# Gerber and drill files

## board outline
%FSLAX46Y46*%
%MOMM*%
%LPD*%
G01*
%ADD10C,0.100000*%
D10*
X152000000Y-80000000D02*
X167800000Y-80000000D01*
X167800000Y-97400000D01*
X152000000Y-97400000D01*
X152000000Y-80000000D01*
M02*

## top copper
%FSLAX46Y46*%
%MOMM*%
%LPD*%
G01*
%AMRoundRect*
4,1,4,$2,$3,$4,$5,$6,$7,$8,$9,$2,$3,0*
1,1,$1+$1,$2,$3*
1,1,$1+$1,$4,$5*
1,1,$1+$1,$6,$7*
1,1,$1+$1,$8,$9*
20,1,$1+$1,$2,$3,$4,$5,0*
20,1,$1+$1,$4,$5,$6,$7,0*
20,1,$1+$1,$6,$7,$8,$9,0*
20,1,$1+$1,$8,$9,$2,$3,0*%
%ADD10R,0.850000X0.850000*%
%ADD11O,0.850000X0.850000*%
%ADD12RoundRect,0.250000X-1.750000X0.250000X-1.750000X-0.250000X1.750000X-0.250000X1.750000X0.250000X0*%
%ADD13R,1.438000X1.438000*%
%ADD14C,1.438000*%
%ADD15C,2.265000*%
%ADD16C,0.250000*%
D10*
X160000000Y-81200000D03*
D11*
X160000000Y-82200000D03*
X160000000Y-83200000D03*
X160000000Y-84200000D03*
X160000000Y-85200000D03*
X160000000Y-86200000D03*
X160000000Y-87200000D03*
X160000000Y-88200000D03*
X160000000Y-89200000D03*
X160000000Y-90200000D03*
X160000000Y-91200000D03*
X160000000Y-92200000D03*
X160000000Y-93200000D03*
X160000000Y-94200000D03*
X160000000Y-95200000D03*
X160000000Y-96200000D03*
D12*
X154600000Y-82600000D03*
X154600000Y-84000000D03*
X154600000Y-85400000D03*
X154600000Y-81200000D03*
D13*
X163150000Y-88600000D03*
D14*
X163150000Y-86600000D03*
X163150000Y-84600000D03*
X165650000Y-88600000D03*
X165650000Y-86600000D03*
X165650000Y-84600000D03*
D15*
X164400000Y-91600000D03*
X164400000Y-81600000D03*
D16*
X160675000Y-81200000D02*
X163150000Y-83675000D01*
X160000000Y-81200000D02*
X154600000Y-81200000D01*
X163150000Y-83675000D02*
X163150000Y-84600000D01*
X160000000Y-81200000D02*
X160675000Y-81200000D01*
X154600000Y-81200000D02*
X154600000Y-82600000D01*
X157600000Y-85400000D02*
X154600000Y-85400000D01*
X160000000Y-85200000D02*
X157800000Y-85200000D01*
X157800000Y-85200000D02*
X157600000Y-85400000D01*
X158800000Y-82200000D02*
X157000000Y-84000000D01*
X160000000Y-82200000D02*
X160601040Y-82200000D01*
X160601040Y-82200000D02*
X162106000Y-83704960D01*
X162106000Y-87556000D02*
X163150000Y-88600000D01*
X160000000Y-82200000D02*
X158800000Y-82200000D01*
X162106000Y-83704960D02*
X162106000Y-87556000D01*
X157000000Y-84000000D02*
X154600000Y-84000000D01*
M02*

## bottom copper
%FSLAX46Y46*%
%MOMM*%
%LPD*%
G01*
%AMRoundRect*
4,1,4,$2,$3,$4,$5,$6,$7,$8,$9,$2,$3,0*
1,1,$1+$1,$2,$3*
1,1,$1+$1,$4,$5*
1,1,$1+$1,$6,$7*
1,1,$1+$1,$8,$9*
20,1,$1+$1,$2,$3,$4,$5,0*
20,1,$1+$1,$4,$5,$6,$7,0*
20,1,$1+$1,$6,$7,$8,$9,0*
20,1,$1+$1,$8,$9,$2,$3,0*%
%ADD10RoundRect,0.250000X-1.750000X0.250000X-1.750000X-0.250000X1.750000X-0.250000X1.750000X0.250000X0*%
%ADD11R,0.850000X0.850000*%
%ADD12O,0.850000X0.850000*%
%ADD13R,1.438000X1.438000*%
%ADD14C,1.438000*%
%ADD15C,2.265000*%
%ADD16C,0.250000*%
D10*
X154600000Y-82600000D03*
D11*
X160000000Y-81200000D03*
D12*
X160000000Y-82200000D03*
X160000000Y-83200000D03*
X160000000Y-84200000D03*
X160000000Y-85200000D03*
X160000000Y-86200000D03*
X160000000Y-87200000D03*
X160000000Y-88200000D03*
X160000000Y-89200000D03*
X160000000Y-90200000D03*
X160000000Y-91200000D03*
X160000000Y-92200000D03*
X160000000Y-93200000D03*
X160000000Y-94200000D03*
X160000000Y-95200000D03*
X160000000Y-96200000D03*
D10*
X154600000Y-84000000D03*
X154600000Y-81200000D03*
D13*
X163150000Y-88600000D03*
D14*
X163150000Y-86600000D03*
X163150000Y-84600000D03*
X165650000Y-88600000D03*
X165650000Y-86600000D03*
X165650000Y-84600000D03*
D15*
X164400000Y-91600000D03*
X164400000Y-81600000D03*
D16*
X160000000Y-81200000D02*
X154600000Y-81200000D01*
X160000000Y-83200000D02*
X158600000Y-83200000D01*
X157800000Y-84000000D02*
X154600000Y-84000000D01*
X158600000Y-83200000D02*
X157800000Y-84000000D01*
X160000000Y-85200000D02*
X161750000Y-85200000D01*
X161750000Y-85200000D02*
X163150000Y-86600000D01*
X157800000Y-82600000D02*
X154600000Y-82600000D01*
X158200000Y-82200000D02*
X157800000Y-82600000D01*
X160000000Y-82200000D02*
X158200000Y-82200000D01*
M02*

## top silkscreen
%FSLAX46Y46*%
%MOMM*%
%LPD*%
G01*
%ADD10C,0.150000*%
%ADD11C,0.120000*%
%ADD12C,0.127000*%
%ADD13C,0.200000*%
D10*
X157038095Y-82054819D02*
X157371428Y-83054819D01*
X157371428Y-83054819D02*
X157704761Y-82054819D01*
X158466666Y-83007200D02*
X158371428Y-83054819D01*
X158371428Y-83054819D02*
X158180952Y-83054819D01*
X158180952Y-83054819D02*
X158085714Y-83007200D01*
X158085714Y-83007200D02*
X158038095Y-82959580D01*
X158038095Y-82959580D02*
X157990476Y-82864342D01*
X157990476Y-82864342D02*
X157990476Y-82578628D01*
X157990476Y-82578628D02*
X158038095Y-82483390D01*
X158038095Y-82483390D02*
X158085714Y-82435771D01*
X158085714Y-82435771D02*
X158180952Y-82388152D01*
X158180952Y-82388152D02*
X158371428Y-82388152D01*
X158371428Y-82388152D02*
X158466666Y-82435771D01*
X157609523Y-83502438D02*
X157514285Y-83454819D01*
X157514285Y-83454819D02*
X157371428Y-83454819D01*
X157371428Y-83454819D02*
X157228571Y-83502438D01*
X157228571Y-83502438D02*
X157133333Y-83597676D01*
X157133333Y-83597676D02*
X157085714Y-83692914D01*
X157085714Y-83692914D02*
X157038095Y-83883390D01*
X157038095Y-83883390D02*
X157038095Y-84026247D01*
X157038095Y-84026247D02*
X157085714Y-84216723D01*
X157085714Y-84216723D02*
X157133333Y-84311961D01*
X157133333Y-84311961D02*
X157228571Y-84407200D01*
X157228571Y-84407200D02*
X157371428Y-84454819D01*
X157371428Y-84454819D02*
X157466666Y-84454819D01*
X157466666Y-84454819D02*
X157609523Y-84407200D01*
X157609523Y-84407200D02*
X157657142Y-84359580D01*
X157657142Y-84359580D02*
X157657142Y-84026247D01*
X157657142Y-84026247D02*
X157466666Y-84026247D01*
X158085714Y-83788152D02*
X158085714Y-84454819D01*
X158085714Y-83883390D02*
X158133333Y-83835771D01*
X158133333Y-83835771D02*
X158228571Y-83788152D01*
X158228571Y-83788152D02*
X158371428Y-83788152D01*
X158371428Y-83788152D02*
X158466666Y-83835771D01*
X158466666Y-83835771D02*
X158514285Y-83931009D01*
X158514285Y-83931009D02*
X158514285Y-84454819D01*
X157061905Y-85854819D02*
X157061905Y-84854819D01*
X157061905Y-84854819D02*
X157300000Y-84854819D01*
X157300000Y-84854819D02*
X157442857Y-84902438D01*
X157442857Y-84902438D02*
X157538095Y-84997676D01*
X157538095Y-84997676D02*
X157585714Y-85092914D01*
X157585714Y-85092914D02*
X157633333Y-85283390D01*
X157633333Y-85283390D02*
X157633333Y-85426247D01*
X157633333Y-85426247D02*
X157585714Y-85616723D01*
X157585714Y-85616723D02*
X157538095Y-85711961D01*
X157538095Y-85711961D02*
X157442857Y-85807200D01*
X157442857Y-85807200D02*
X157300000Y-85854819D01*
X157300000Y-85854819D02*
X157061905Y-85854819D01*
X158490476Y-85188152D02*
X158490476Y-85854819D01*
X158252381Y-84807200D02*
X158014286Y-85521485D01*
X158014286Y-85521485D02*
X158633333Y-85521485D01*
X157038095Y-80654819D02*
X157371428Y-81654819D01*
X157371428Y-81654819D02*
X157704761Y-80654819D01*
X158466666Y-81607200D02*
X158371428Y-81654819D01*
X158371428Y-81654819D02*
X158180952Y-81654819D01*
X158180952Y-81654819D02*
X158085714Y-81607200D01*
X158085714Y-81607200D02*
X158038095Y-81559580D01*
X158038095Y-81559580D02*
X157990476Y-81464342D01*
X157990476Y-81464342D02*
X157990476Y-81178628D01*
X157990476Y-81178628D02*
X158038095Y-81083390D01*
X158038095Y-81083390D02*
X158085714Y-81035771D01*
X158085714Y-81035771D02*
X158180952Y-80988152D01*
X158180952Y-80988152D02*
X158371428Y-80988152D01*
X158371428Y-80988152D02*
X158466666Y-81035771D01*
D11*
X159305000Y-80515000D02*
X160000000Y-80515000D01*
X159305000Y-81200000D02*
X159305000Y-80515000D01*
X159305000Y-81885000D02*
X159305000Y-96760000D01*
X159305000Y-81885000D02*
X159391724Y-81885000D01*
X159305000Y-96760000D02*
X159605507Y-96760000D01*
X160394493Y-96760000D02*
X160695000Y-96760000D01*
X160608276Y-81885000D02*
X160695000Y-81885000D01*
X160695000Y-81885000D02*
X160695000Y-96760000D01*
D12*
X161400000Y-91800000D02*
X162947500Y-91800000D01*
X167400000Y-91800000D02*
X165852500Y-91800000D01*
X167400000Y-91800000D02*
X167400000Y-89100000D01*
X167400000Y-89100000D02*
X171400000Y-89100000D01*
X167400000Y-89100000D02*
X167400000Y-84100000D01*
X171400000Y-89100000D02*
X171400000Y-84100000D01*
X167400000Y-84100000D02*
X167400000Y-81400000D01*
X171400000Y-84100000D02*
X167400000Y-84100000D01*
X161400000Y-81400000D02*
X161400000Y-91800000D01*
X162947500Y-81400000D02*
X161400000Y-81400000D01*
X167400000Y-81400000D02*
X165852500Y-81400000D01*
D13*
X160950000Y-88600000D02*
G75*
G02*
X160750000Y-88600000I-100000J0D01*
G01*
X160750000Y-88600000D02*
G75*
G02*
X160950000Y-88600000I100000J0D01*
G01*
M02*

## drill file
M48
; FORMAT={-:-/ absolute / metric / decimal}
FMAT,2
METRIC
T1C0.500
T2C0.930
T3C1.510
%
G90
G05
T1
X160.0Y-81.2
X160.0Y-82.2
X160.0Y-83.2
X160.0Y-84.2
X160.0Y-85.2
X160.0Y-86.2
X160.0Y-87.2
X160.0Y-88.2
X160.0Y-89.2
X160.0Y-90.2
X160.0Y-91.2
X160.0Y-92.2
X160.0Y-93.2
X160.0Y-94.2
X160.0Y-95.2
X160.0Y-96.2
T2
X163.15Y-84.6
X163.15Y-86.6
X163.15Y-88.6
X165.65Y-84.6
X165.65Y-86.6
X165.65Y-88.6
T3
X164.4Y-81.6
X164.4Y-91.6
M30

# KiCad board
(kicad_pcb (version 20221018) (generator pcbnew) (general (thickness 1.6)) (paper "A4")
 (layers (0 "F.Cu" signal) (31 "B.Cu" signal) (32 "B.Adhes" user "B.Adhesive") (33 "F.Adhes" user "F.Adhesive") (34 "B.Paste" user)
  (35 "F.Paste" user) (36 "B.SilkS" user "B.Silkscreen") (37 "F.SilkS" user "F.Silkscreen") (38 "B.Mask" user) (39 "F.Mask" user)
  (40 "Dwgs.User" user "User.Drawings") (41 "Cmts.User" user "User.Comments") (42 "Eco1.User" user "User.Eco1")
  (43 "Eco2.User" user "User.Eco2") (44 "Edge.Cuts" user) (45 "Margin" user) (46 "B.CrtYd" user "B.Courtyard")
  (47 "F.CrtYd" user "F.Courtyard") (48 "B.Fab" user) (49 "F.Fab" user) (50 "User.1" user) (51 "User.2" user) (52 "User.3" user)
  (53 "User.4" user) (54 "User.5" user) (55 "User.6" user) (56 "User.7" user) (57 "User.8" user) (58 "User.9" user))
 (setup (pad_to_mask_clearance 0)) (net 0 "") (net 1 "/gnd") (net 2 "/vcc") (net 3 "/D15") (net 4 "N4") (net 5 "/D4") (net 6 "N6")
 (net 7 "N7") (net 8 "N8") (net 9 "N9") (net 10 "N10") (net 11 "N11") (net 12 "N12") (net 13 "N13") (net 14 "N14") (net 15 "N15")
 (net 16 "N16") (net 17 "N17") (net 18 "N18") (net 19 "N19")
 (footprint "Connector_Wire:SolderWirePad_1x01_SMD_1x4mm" (layer "F.Cu") (at 154.6 82.6 -90)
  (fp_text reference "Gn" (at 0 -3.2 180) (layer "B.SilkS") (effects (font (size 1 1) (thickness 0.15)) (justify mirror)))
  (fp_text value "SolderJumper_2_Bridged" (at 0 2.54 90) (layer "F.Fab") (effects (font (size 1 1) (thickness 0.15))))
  (pad "1" smd roundrect (at 0 0 270) (size 1 4) (layers "B.Cu" "B.Paste" "B.Mask") (roundrect_rratio 0.25) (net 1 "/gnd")))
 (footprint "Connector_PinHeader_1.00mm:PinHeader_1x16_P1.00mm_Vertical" (layer "F.Cu") (at 160 81.2)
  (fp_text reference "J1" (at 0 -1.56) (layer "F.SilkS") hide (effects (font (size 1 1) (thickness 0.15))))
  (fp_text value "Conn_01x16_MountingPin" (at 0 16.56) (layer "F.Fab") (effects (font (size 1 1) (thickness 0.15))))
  (fp_line (start -0.695 -0.685) (end 0 -0.685) (stroke (width 0.12) (type solid)) (layer "F.SilkS"))
  (fp_line (start -0.695 0) (end -0.695 -0.685) (stroke (width 0.12) (type solid)) (layer "F.SilkS"))
  (fp_line (start -0.695 0.685) (end -0.695 15.56) (stroke (width 0.12) (type solid)) (layer "F.SilkS"))
  (fp_line (start -0.695 0.685) (end -0.608276 0.685) (stroke (width 0.12) (type solid)) (layer "F.SilkS"))
  (fp_line (start -0.695 15.56) (end -0.394493 15.56) (stroke (width 0.12) (type solid)) (layer "F.SilkS"))
  (fp_line (start 0.394493 15.56) (end 0.695 15.56) (stroke (width 0.12) (type solid)) (layer "F.SilkS"))
  (fp_line (start 0.608276 0.685) (end 0.695 0.685) (stroke (width 0.12) (type solid)) (layer "F.SilkS"))
  (fp_line (start 0.695 0.685) (end 0.695 15.56) (stroke (width 0.12) (type solid)) (layer "F.SilkS"))
  (pad "1" thru_hole rect (at 0 0) (size 0.85 0.85) (drill 0.5) (layers "*.Cu" "*.Mask") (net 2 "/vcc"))
  (pad "2" thru_hole oval (at 0 1) (size 0.85 0.85) (drill 0.5) (layers "*.Cu" "*.Mask") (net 1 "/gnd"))
  (pad "3" thru_hole oval (at 0 2) (size 0.85 0.85) (drill 0.5) (layers "*.Cu" "*.Mask") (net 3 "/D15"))
  (pad "4" thru_hole oval (at 0 3) (size 0.85 0.85) (drill 0.5) (layers "*.Cu" "*.Mask") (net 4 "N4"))
  (pad "5" thru_hole oval (at 0 4) (size 0.85 0.85) (drill 0.5) (layers "*.Cu" "*.Mask") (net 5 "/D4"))
  (pad "6" thru_hole oval (at 0 5) (size 0.85 0.85) (drill 0.5) (layers "*.Cu" "*.Mask") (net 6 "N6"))
  (pad "7" thru_hole oval (at 0 6) (size 0.85 0.85) (drill 0.5) (layers "*.Cu" "*.Mask") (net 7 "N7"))
  (pad "8" thru_hole oval (at 0 7) (size 0.85 0.85) (drill 0.5) (layers "*.Cu" "*.Mask") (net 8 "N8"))
  (pad "9" thru_hole oval (at 0 8) (size 0.85 0.85) (drill 0.5) (layers "*.Cu" "*.Mask") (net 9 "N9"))
  (pad "10" thru_hole oval (at 0 9) (size 0.85 0.85) (drill 0.5) (layers "*.Cu" "*.Mask") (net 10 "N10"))
  (pad "11" thru_hole oval (at 0 10) (size 0.85 0.85) (drill 0.5) (layers "*.Cu" "*.Mask") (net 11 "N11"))
  (pad "12" thru_hole oval (at 0 11) (size 0.85 0.85) (drill 0.5) (layers "*.Cu" "*.Mask") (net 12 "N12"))
  (pad "13" thru_hole oval (at 0 12) (size 0.85 0.85) (drill 0.5) (layers "*.Cu" "*.Mask") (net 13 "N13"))
  (pad "14" thru_hole oval (at 0 13) (size 0.85 0.85) (drill 0.5) (layers "*.Cu" "*.Mask") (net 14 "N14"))
  (pad "15" thru_hole oval (at 0 14) (size 0.85 0.85) (drill 0.5) (layers "*.Cu" "*.Mask") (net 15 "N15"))
  (pad "16" thru_hole oval (at 0 15) (size 0.85 0.85) (drill 0.5) (layers "*.Cu" "*.Mask") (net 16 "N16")))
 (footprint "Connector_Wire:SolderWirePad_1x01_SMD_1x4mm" (layer "F.Cu") (at 154.6 82.6 -90)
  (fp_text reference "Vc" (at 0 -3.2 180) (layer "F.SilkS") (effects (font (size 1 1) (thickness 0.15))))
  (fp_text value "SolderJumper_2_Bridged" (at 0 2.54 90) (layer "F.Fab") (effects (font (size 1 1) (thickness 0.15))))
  (pad "1" smd roundrect (at 0 0 270) (size 1 4) (layers "F.Cu" "F.Paste" "F.Mask") (roundrect_rratio 0.25) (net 2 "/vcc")))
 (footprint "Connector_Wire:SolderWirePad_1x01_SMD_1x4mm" (layer "F.Cu") (at 154.6 84 -90)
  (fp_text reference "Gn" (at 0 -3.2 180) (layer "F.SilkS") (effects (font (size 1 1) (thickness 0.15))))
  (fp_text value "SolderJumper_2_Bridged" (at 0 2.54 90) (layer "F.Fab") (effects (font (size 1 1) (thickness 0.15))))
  (pad "1" smd roundrect (at 0 0 270) (size 1 4) (layers "F.Cu" "F.Paste" "F.Mask") (roundrect_rratio 0.25) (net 1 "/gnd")))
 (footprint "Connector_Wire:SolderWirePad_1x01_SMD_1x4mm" (layer "F.Cu") (at 154.6 84 -90)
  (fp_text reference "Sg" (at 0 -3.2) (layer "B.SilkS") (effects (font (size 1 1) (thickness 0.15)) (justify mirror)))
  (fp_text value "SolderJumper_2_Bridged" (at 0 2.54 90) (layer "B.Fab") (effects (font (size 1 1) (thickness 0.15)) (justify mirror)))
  (pad "1" smd roundrect (at 0 0 270) (size 1 4) (layers "B.Cu" "B.Paste" "B.Mask") (roundrect_rratio 0.25) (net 3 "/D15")))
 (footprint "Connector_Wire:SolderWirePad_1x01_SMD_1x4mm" (layer "F.Cu") (at 154.6 81.2 -90)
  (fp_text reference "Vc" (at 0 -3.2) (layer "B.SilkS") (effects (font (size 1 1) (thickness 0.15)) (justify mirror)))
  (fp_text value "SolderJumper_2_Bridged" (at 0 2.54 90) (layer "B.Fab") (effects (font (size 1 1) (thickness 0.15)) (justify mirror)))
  (pad "1" smd roundrect (at 0 0 270) (size 1 4) (layers "B.Cu" "B.Paste" "B.Mask") (roundrect_rratio 0.25) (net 2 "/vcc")))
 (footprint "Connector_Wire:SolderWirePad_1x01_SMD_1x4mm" (layer "F.Cu") (at 154.6 85.4 -90)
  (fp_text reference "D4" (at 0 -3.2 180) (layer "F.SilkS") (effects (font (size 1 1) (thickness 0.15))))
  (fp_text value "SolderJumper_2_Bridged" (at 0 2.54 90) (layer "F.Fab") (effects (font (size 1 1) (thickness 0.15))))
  (pad "1" smd roundrect (at 0 0 270) (size 1 4) (layers "F.Cu" "F.Paste" "F.Mask") (roundrect_rratio 0.25) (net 5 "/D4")))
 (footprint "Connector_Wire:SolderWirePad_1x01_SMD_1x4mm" (layer "F.Cu") (at 154.6 81.2 -90)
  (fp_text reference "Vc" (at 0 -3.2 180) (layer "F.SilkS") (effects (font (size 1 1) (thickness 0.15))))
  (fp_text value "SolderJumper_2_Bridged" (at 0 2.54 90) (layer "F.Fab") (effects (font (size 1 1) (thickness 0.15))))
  (pad "1" smd roundrect (at 0 0 270) (size 1 4) (layers "F.Cu" "F.Paste" "F.Mask") (roundrect_rratio 0.25) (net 2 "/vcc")))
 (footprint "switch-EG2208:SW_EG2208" (layer "F.Cu") (at 164.4 86.6 90)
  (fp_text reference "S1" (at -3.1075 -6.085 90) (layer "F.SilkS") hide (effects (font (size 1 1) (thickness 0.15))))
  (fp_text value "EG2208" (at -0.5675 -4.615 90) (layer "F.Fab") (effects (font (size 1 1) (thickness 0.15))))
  (fp_line (start -5.2 -3) (end -5.2 -1.4525) (stroke (width 0.127) (type solid)) (layer "F.SilkS"))
  (fp_line (start -5.2 3) (end -5.2 1.4525) (stroke (width 0.127) (type solid)) (layer "F.SilkS"))
  (fp_line (start -5.2 3) (end -2.5 3) (stroke (width 0.127) (type solid)) (layer "F.SilkS"))
  (fp_line (start -2.5 3) (end -2.5 7) (stroke (width 0.127) (type solid)) (layer "F.SilkS"))
  (fp_line (start -2.5 3) (end 2.5 3) (stroke (width 0.127) (type solid)) (layer "F.SilkS"))
  (fp_line (start -2.5 7) (end 2.5 7) (stroke (width 0.127) (type solid)) (layer "F.SilkS"))
  (fp_line (start 2.5 3) (end 5.2 3) (stroke (width 0.127) (type solid)) (layer "F.SilkS"))
  (fp_line (start 2.5 7) (end 2.5 3) (stroke (width 0.127) (type solid)) (layer "F.SilkS"))
  (fp_line (start 5.2 -3) (end -5.2 -3) (stroke (width 0.127) (type solid)) (layer "F.SilkS"))
  (fp_line (start 5.2 -1.4525) (end 5.2 -3) (stroke (width 0.127) (type solid)) (layer "F.SilkS"))
  (fp_line (start 5.2 3) (end 5.2 1.4525) (stroke (width 0.127) (type solid)) (layer "F.SilkS"))
  (fp_circle (center -2 -3.55) (end -1.9 -3.55) (stroke (width 0.2) (type solid)) (fill none) (layer "F.SilkS"))
  (pad "1" thru_hole rect (at -2 -1.25 90) (size 1.438 1.438) (drill 0.93) (layers "*.Cu" "*.Mask") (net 1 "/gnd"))
  (pad "2" thru_hole circle (at 0 -1.25 90) (size 1.438 1.438) (drill 0.93) (layers "*.Cu" "*.Mask") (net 5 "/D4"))
  (pad "3" thru_hole circle (at 2 -1.25 90) (size 1.438 1.438) (drill 0.93) (layers "*.Cu" "*.Mask") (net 2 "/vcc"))
  (pad "4" thru_hole circle (at -2 1.25 90) (size 1.438 1.438) (drill 0.93) (layers "*.Cu" "*.Mask") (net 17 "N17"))
  (pad "5" thru_hole circle (at 0 1.25 90) (size 1.438 1.438) (drill 0.93) (layers "*.Cu" "*.Mask") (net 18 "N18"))
  (pad "6" thru_hole circle (at 2 1.25 90) (size 1.438 1.438) (drill 0.93) (layers "*.Cu" "*.Mask") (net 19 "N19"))
  (pad "S1" thru_hole circle (at -5 0 90) (size 2.265 2.265) (drill 1.51) (layers "*.Cu" "*.Mask"))
  (pad "S2" thru_hole circle (at 5 0 90) (size 2.265 2.265) (drill 1.51) (layers "*.Cu" "*.Mask")))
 (gr_rect (start 152 80) (end 167.8 97.4) (stroke (width 0.1) (type default)) (fill none) (layer "Edge.Cuts"))
 (segment (start 160.675 81.2) (end 163.15 83.675) (width 0.25) (layer "F.Cu") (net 2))
 (segment (start 160 81.2) (end 154.6 81.2) (width 0.25) (layer "F.Cu") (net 2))
 (segment (start 163.15 83.675) (end 163.15 84.6) (width 0.25) (layer "F.Cu") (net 2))
 (segment (start 160 81.2) (end 160.675 81.2) (width 0.25) (layer "F.Cu") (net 2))
 (segment (start 154.6 81.2) (end 154.6 82.6) (width 0.25) (layer "F.Cu") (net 2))
 (segment (start 160 81.2) (end 154.6 81.2) (width 0.25) (layer "B.Cu") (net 2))
 (segment (start 160 83.2) (end 158.6 83.2) (width 0.25) (layer "B.Cu") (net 3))
 (segment (start 157.8 84) (end 154.6 84) (width 0.25) (layer "B.Cu") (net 3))
 (segment (start 158.6 83.2) (end 157.8 84) (width 0.25) (layer "B.Cu") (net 3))
 (segment (start 157.6 85.4) (end 154.6 85.4) (width 0.25) (layer "F.Cu") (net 5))
 (segment (start 160 85.2) (end 157.8 85.2) (width 0.25) (layer "F.Cu") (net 5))
 (segment (start 157.8 85.2) (end 157.6 85.4) (width 0.25) (layer "F.Cu") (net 5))
 (segment (start 160 85.2) (end 161.75 85.2) (width 0.25) (layer "B.Cu") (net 5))
 (segment (start 161.75 85.2) (end 163.15 86.6) (width 0.25) (layer "B.Cu") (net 5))
 (segment (start 158.8 82.2) (end 157 84) (width 0.25) (layer "F.Cu") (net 1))
 (segment (start 160 82.2) (end 160.60104 82.2) (width 0.25) (layer "F.Cu") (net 1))
 (segment (start 160.60104 82.2) (end 162.106 83.70496) (width 0.25) (layer "F.Cu") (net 1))
 (segment (start 162.106 87.556) (end 163.15 88.6) (width 0.25) (layer "F.Cu") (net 1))
 (segment (start 160 82.2) (end 158.8 82.2) (width 0.25) (layer "F.Cu") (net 1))
 (segment (start 162.106 83.70496) (end 162.106 87.556) (width 0.25) (layer "F.Cu") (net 1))
 (segment (start 157 84) (end 154.6 84) (width 0.25) (layer "F.Cu") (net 1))
 (segment (start 157.8 82.6) (end 154.6 82.6) (width 0.25) (layer "B.Cu") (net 1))
 (segment (start 158.2 82.2) (end 157.8 82.6) (width 0.25) (layer "B.Cu") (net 1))
 (segment (start 160 82.2) (end 158.2 82.2) (width 0.25) (layer "B.Cu") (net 1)))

